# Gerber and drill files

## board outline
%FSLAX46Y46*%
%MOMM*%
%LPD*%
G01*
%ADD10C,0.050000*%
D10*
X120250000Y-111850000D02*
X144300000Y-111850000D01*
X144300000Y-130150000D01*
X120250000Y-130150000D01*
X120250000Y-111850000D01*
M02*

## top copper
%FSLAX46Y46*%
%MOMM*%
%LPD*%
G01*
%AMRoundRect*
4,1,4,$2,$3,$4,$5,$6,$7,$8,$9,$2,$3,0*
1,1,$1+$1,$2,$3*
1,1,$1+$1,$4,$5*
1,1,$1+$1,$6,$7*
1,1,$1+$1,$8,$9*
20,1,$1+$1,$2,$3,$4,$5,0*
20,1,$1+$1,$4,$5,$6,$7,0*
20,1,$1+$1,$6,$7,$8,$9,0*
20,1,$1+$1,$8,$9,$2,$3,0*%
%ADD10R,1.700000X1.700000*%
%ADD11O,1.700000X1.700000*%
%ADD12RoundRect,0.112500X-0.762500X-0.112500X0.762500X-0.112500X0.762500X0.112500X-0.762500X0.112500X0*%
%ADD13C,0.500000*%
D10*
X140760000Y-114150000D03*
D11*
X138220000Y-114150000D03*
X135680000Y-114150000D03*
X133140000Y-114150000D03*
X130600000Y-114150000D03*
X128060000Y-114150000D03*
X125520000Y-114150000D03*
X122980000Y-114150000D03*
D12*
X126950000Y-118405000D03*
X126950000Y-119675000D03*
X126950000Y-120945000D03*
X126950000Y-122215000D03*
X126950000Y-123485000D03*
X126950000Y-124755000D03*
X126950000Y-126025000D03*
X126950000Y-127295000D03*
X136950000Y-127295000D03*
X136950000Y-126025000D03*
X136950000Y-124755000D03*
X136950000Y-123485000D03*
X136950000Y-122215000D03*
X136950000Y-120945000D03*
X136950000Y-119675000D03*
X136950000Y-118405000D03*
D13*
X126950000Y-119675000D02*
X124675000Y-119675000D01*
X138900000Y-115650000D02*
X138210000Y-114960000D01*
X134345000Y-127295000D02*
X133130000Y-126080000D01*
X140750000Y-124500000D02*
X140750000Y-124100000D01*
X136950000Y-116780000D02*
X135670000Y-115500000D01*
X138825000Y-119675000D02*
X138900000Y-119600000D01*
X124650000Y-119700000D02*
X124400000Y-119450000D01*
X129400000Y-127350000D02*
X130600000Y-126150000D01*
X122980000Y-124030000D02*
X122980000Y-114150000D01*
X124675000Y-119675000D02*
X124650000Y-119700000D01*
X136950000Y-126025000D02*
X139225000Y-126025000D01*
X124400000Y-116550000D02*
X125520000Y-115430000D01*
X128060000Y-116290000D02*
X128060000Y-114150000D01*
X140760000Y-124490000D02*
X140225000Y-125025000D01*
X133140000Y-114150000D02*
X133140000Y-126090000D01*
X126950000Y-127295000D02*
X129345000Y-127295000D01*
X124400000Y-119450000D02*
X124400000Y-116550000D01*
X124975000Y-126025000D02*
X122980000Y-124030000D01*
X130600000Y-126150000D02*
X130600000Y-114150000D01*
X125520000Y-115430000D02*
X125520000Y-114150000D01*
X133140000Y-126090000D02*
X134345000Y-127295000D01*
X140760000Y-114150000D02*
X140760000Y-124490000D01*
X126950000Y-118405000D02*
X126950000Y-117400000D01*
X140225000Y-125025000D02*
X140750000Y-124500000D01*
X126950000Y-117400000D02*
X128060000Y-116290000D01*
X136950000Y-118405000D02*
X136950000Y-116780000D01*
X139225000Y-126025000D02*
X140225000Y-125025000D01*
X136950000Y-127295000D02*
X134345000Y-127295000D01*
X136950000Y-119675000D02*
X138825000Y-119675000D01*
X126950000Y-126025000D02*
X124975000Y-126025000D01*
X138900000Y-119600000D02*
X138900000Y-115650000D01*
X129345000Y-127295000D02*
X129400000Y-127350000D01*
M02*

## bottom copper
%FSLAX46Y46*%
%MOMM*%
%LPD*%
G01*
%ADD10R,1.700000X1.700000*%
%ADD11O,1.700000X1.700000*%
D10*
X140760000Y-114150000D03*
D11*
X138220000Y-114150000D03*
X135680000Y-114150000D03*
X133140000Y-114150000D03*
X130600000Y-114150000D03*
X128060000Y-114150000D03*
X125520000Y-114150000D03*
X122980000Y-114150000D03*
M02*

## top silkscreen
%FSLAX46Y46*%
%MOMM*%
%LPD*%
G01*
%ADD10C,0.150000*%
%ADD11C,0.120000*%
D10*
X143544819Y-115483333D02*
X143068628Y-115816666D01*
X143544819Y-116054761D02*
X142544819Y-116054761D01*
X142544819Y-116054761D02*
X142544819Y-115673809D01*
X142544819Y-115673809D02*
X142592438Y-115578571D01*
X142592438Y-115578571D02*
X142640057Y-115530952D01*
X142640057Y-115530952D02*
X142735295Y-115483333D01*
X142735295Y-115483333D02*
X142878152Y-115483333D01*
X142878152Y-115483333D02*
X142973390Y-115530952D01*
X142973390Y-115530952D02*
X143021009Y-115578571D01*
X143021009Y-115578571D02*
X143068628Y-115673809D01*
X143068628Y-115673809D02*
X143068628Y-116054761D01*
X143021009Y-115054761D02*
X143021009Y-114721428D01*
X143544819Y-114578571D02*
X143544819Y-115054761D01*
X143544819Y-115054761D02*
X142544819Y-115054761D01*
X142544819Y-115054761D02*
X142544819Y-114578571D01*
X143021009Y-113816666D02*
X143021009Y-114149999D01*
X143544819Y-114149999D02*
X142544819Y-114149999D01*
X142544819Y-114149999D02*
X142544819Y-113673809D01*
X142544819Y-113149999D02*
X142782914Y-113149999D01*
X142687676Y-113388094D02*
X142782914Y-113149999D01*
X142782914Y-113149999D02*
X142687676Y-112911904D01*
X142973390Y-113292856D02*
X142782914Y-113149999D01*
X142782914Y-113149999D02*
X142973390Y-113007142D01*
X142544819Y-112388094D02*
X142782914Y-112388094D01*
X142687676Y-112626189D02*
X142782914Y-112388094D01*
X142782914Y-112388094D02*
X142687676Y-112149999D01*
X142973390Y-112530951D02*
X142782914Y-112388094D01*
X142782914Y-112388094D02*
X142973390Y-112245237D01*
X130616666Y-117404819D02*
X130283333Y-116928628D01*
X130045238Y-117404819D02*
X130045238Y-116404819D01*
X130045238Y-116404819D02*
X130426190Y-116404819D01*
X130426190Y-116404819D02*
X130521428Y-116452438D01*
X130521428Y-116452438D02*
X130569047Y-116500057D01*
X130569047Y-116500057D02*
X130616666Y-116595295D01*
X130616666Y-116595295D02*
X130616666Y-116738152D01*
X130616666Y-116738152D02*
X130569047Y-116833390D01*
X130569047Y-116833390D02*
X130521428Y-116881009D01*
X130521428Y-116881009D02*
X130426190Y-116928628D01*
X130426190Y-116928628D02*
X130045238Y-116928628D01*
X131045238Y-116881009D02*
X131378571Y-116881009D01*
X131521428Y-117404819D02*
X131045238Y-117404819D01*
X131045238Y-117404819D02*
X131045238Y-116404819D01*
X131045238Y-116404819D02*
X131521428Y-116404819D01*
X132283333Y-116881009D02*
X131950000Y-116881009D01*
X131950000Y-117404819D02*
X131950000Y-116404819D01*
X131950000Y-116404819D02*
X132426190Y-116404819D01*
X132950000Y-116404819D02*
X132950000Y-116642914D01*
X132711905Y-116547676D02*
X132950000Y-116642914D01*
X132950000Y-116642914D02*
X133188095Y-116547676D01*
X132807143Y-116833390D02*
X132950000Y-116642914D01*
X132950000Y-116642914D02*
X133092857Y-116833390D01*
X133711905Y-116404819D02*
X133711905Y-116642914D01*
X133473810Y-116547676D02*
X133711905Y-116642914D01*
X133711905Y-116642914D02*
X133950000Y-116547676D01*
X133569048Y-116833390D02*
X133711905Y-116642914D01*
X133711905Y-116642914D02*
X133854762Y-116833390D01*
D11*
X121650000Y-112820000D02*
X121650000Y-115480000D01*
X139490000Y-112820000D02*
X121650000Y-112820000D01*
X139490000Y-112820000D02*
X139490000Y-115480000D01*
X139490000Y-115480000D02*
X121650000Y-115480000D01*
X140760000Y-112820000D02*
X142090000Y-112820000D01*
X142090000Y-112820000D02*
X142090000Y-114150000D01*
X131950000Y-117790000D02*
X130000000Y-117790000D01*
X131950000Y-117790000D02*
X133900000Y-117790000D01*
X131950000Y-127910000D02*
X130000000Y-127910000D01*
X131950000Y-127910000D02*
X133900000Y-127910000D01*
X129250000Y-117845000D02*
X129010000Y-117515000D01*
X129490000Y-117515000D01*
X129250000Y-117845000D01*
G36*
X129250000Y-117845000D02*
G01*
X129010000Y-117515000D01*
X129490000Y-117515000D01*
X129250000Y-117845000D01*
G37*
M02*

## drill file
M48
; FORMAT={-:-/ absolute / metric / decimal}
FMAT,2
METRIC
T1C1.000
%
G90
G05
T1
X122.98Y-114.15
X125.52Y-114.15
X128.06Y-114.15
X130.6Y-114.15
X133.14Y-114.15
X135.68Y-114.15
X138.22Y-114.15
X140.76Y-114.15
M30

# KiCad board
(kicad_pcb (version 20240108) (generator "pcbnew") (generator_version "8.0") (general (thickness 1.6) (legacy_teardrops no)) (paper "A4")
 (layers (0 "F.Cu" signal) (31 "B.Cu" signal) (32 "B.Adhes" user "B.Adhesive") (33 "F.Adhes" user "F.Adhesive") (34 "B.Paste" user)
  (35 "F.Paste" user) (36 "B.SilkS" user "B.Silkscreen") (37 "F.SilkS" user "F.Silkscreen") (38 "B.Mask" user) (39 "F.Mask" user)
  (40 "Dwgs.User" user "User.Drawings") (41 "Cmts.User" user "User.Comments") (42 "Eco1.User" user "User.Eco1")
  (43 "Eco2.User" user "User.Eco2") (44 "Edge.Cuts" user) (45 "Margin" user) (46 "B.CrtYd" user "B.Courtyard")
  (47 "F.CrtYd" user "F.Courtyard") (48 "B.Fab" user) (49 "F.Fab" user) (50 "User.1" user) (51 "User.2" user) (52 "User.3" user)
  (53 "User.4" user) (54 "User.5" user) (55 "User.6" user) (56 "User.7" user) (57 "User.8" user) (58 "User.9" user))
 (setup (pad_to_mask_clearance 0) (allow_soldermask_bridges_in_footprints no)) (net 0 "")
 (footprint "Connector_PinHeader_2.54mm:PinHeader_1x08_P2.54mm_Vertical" (layer "F.Cu") (at 140.76 114.15 -90)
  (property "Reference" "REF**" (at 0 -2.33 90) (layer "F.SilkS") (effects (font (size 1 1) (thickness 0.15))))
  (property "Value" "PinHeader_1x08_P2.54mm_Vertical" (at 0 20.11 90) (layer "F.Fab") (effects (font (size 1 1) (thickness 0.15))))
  (fp_line (start -1.33 19.11) (end 1.33 19.11) (stroke (width 0.12) (type solid)) (layer "F.SilkS"))
  (fp_line (start -1.33 1.27) (end -1.33 19.11) (stroke (width 0.12) (type solid)) (layer "F.SilkS"))
  (fp_line (start -1.33 1.27) (end 1.33 1.27) (stroke (width 0.12) (type solid)) (layer "F.SilkS"))
  (fp_line (start 1.33 1.27) (end 1.33 19.11) (stroke (width 0.12) (type solid)) (layer "F.SilkS"))
  (fp_line (start -1.33 0) (end -1.33 -1.33) (stroke (width 0.12) (type solid)) (layer "F.SilkS"))
  (fp_line (start -1.33 -1.33) (end 0 -1.33) (stroke (width 0.12) (type solid)) (layer "F.SilkS"))
  (pad "1" thru_hole rect (at 0 0 270) (size 1.7 1.7) (drill 1) (layers "*.Cu" "*.Mask") (remove_unused_layers no))
  (pad "2" thru_hole oval (at 0 2.54 270) (size 1.7 1.7) (drill 1) (layers "*.Cu" "*.Mask") (remove_unused_layers no))
  (pad "3" thru_hole oval (at 0 5.08 270) (size 1.7 1.7) (drill 1) (layers "*.Cu" "*.Mask") (remove_unused_layers no))
  (pad "4" thru_hole oval (at 0 7.62 270) (size 1.7 1.7) (drill 1) (layers "*.Cu" "*.Mask") (remove_unused_layers no))
  (pad "5" thru_hole oval (at 0 10.16 270) (size 1.7 1.7) (drill 1) (layers "*.Cu" "*.Mask") (remove_unused_layers no))
  (pad "6" thru_hole oval (at 0 12.7 270) (size 1.7 1.7) (drill 1) (layers "*.Cu" "*.Mask") (remove_unused_layers no))
  (pad "7" thru_hole oval (at 0 15.24 270) (size 1.7 1.7) (drill 1) (layers "*.Cu" "*.Mask") (remove_unused_layers no))
  (pad "8" thru_hole oval (at 0 17.78 270) (size 1.7 1.7) (drill 1) (layers "*.Cu" "*.Mask") (remove_unused_layers no)))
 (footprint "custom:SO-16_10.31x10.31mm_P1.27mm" (layer "F.Cu") (at 131.95 122.85)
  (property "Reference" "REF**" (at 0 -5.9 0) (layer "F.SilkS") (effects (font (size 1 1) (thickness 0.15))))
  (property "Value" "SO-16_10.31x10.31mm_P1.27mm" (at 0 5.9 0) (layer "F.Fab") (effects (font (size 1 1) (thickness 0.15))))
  (fp_line (start 0 -5.06) (end -1.95 -5.06) (stroke (width 0.12) (type solid)) (layer "F.SilkS"))
  (fp_line (start 0 -5.06) (end 1.95 -5.06) (stroke (width 0.12) (type solid)) (layer "F.SilkS"))
  (fp_line (start 0 5.06) (end -1.95 5.06) (stroke (width 0.12) (type solid)) (layer "F.SilkS"))
  (fp_line (start 0 5.06) (end 1.95 5.06) (stroke (width 0.12) (type solid)) (layer "F.SilkS"))
  (fp_poly
   (pts (xy -2.7 -5.005) (xy -2.94 -5.335) (xy -2.46 -5.335) (xy -2.7 -5.005)) (stroke (width 0.12) (type solid)) (fill solid)
   (layer "F.SilkS"))
  (pad "1" smd roundrect (at -5 -4.445) (size 1.75 0.45) (layers "F.Cu" "F.Paste" "F.Mask") (roundrect_rratio 0.25))
  (pad "2" smd roundrect (at -5 -3.175) (size 1.75 0.45) (layers "F.Cu" "F.Paste" "F.Mask") (roundrect_rratio 0.25))
  (pad "3" smd roundrect (at -5 -1.905) (size 1.75 0.45) (layers "F.Cu" "F.Paste" "F.Mask") (roundrect_rratio 0.25))
  (pad "4" smd roundrect (at -5 -0.635) (size 1.75 0.45) (layers "F.Cu" "F.Paste" "F.Mask") (roundrect_rratio 0.25))
  (pad "5" smd roundrect (at -5 0.635) (size 1.75 0.45) (layers "F.Cu" "F.Paste" "F.Mask") (roundrect_rratio 0.25))
  (pad "6" smd roundrect (at -5 1.905) (size 1.75 0.45) (layers "F.Cu" "F.Paste" "F.Mask") (roundrect_rratio 0.25))
  (pad "7" smd roundrect (at -5 3.175) (size 1.75 0.45) (layers "F.Cu" "F.Paste" "F.Mask") (roundrect_rratio 0.25))
  (pad "8" smd roundrect (at -5 4.445) (size 1.75 0.45) (layers "F.Cu" "F.Paste" "F.Mask") (roundrect_rratio 0.25))
  (pad "9" smd roundrect (at 5 4.445) (size 1.75 0.45) (layers "F.Cu" "F.Paste" "F.Mask") (roundrect_rratio 0.25))
  (pad "10" smd roundrect (at 5 3.175) (size 1.75 0.45) (layers "F.Cu" "F.Paste" "F.Mask") (roundrect_rratio 0.25))
  (pad "11" smd roundrect (at 5 1.905) (size 1.75 0.45) (layers "F.Cu" "F.Paste" "F.Mask") (roundrect_rratio 0.25))
  (pad "12" smd roundrect (at 5 0.635) (size 1.75 0.45) (layers "F.Cu" "F.Paste" "F.Mask") (roundrect_rratio 0.25))
  (pad "13" smd roundrect (at 5 -0.635) (size 1.75 0.45) (layers "F.Cu" "F.Paste" "F.Mask") (roundrect_rratio 0.25))
  (pad "14" smd roundrect (at 5 -1.905) (size 1.75 0.45) (layers "F.Cu" "F.Paste" "F.Mask") (roundrect_rratio 0.25))
  (pad "15" smd roundrect (at 5 -3.175) (size 1.75 0.45) (layers "F.Cu" "F.Paste" "F.Mask") (roundrect_rratio 0.25))
  (pad "16" smd roundrect (at 5 -4.445) (size 1.75 0.45) (layers "F.Cu" "F.Paste" "F.Mask") (roundrect_rratio 0.25)))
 (gr_rect (start 120.25 111.85) (end 144.3 130.15) (stroke (width 0.05) (type default)) (fill none) (layer "Edge.Cuts"))
 (segment (start 126.95 119.675) (end 124.675 119.675) (width 0.5) (layer "F.Cu") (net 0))
 (segment (start 138.9 115.65) (end 138.21 114.96) (width 0.5) (layer "F.Cu") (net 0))
 (segment (start 134.345 127.295) (end 133.13 126.08) (width 0.5) (layer "F.Cu") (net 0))
 (segment (start 140.75 124.5) (end 140.75 124.1) (width 0.5) (layer "F.Cu") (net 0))
 (segment (start 136.95 116.78) (end 135.67 115.5) (width 0.5) (layer "F.Cu") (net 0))
 (segment (start 138.825 119.675) (end 138.9 119.6) (width 0.5) (layer "F.Cu") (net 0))
 (segment (start 124.65 119.7) (end 124.4 119.45) (width 0.5) (layer "F.Cu") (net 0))
 (segment (start 129.4 127.35) (end 130.6 126.15) (width 0.5) (layer "F.Cu") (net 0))
 (segment (start 122.98 124.03) (end 122.98 114.15) (width 0.5) (layer "F.Cu") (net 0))
 (segment (start 124.675 119.675) (end 124.65 119.7) (width 0.5) (layer "F.Cu") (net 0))
 (segment (start 136.95 126.025) (end 139.225 126.025) (width 0.5) (layer "F.Cu") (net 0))
 (segment (start 124.4 116.55) (end 125.52 115.43) (width 0.5) (layer "F.Cu") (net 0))
 (segment (start 128.06 116.29) (end 128.06 114.15) (width 0.5) (layer "F.Cu") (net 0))
 (segment (start 140.76 124.49) (end 140.225 125.025) (width 0.5) (layer "F.Cu") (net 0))
 (segment (start 133.14 114.15) (end 133.14 126.09) (width 0.5) (layer "F.Cu") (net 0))
 (segment (start 126.95 127.295) (end 129.345 127.295) (width 0.5) (layer "F.Cu") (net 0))
 (segment (start 124.4 119.45) (end 124.4 116.55) (width 0.5) (layer "F.Cu") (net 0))
 (segment (start 124.975 126.025) (end 122.98 124.03) (width 0.5) (layer "F.Cu") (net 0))
 (segment (start 130.6 126.15) (end 130.6 114.15) (width 0.5) (layer "F.Cu") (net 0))
 (segment (start 125.52 115.43) (end 125.52 114.15) (width 0.5) (layer "F.Cu") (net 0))
 (segment (start 133.14 126.09) (end 134.345 127.295) (width 0.5) (layer "F.Cu") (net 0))
 (segment (start 140.76 114.15) (end 140.76 124.49) (width 0.5) (layer "F.Cu") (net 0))
 (segment (start 126.95 118.405) (end 126.95 117.4) (width 0.5) (layer "F.Cu") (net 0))
 (segment (start 140.225 125.025) (end 140.75 124.5) (width 0.5) (layer "F.Cu") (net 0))
 (segment (start 126.95 117.4) (end 128.06 116.29) (width 0.5) (layer "F.Cu") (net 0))
 (segment (start 136.95 118.405) (end 136.95 116.78) (width 0.5) (layer "F.Cu") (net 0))
 (segment (start 139.225 126.025) (end 140.225 125.025) (width 0.5) (layer "F.Cu") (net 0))
 (segment (start 136.95 127.295) (end 134.345 127.295) (width 0.5) (layer "F.Cu") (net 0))
 (segment (start 136.95 119.675) (end 138.825 119.675) (width 0.5) (layer "F.Cu") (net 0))
 (segment (start 126.95 126.025) (end 124.975 126.025) (width 0.5) (layer "F.Cu") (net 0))
 (segment (start 138.9 119.6) (end 138.9 115.65) (width 0.5) (layer "F.Cu") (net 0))
 (segment (start 129.345 127.295) (end 129.4 127.35) (width 0.5) (layer "F.Cu") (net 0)))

